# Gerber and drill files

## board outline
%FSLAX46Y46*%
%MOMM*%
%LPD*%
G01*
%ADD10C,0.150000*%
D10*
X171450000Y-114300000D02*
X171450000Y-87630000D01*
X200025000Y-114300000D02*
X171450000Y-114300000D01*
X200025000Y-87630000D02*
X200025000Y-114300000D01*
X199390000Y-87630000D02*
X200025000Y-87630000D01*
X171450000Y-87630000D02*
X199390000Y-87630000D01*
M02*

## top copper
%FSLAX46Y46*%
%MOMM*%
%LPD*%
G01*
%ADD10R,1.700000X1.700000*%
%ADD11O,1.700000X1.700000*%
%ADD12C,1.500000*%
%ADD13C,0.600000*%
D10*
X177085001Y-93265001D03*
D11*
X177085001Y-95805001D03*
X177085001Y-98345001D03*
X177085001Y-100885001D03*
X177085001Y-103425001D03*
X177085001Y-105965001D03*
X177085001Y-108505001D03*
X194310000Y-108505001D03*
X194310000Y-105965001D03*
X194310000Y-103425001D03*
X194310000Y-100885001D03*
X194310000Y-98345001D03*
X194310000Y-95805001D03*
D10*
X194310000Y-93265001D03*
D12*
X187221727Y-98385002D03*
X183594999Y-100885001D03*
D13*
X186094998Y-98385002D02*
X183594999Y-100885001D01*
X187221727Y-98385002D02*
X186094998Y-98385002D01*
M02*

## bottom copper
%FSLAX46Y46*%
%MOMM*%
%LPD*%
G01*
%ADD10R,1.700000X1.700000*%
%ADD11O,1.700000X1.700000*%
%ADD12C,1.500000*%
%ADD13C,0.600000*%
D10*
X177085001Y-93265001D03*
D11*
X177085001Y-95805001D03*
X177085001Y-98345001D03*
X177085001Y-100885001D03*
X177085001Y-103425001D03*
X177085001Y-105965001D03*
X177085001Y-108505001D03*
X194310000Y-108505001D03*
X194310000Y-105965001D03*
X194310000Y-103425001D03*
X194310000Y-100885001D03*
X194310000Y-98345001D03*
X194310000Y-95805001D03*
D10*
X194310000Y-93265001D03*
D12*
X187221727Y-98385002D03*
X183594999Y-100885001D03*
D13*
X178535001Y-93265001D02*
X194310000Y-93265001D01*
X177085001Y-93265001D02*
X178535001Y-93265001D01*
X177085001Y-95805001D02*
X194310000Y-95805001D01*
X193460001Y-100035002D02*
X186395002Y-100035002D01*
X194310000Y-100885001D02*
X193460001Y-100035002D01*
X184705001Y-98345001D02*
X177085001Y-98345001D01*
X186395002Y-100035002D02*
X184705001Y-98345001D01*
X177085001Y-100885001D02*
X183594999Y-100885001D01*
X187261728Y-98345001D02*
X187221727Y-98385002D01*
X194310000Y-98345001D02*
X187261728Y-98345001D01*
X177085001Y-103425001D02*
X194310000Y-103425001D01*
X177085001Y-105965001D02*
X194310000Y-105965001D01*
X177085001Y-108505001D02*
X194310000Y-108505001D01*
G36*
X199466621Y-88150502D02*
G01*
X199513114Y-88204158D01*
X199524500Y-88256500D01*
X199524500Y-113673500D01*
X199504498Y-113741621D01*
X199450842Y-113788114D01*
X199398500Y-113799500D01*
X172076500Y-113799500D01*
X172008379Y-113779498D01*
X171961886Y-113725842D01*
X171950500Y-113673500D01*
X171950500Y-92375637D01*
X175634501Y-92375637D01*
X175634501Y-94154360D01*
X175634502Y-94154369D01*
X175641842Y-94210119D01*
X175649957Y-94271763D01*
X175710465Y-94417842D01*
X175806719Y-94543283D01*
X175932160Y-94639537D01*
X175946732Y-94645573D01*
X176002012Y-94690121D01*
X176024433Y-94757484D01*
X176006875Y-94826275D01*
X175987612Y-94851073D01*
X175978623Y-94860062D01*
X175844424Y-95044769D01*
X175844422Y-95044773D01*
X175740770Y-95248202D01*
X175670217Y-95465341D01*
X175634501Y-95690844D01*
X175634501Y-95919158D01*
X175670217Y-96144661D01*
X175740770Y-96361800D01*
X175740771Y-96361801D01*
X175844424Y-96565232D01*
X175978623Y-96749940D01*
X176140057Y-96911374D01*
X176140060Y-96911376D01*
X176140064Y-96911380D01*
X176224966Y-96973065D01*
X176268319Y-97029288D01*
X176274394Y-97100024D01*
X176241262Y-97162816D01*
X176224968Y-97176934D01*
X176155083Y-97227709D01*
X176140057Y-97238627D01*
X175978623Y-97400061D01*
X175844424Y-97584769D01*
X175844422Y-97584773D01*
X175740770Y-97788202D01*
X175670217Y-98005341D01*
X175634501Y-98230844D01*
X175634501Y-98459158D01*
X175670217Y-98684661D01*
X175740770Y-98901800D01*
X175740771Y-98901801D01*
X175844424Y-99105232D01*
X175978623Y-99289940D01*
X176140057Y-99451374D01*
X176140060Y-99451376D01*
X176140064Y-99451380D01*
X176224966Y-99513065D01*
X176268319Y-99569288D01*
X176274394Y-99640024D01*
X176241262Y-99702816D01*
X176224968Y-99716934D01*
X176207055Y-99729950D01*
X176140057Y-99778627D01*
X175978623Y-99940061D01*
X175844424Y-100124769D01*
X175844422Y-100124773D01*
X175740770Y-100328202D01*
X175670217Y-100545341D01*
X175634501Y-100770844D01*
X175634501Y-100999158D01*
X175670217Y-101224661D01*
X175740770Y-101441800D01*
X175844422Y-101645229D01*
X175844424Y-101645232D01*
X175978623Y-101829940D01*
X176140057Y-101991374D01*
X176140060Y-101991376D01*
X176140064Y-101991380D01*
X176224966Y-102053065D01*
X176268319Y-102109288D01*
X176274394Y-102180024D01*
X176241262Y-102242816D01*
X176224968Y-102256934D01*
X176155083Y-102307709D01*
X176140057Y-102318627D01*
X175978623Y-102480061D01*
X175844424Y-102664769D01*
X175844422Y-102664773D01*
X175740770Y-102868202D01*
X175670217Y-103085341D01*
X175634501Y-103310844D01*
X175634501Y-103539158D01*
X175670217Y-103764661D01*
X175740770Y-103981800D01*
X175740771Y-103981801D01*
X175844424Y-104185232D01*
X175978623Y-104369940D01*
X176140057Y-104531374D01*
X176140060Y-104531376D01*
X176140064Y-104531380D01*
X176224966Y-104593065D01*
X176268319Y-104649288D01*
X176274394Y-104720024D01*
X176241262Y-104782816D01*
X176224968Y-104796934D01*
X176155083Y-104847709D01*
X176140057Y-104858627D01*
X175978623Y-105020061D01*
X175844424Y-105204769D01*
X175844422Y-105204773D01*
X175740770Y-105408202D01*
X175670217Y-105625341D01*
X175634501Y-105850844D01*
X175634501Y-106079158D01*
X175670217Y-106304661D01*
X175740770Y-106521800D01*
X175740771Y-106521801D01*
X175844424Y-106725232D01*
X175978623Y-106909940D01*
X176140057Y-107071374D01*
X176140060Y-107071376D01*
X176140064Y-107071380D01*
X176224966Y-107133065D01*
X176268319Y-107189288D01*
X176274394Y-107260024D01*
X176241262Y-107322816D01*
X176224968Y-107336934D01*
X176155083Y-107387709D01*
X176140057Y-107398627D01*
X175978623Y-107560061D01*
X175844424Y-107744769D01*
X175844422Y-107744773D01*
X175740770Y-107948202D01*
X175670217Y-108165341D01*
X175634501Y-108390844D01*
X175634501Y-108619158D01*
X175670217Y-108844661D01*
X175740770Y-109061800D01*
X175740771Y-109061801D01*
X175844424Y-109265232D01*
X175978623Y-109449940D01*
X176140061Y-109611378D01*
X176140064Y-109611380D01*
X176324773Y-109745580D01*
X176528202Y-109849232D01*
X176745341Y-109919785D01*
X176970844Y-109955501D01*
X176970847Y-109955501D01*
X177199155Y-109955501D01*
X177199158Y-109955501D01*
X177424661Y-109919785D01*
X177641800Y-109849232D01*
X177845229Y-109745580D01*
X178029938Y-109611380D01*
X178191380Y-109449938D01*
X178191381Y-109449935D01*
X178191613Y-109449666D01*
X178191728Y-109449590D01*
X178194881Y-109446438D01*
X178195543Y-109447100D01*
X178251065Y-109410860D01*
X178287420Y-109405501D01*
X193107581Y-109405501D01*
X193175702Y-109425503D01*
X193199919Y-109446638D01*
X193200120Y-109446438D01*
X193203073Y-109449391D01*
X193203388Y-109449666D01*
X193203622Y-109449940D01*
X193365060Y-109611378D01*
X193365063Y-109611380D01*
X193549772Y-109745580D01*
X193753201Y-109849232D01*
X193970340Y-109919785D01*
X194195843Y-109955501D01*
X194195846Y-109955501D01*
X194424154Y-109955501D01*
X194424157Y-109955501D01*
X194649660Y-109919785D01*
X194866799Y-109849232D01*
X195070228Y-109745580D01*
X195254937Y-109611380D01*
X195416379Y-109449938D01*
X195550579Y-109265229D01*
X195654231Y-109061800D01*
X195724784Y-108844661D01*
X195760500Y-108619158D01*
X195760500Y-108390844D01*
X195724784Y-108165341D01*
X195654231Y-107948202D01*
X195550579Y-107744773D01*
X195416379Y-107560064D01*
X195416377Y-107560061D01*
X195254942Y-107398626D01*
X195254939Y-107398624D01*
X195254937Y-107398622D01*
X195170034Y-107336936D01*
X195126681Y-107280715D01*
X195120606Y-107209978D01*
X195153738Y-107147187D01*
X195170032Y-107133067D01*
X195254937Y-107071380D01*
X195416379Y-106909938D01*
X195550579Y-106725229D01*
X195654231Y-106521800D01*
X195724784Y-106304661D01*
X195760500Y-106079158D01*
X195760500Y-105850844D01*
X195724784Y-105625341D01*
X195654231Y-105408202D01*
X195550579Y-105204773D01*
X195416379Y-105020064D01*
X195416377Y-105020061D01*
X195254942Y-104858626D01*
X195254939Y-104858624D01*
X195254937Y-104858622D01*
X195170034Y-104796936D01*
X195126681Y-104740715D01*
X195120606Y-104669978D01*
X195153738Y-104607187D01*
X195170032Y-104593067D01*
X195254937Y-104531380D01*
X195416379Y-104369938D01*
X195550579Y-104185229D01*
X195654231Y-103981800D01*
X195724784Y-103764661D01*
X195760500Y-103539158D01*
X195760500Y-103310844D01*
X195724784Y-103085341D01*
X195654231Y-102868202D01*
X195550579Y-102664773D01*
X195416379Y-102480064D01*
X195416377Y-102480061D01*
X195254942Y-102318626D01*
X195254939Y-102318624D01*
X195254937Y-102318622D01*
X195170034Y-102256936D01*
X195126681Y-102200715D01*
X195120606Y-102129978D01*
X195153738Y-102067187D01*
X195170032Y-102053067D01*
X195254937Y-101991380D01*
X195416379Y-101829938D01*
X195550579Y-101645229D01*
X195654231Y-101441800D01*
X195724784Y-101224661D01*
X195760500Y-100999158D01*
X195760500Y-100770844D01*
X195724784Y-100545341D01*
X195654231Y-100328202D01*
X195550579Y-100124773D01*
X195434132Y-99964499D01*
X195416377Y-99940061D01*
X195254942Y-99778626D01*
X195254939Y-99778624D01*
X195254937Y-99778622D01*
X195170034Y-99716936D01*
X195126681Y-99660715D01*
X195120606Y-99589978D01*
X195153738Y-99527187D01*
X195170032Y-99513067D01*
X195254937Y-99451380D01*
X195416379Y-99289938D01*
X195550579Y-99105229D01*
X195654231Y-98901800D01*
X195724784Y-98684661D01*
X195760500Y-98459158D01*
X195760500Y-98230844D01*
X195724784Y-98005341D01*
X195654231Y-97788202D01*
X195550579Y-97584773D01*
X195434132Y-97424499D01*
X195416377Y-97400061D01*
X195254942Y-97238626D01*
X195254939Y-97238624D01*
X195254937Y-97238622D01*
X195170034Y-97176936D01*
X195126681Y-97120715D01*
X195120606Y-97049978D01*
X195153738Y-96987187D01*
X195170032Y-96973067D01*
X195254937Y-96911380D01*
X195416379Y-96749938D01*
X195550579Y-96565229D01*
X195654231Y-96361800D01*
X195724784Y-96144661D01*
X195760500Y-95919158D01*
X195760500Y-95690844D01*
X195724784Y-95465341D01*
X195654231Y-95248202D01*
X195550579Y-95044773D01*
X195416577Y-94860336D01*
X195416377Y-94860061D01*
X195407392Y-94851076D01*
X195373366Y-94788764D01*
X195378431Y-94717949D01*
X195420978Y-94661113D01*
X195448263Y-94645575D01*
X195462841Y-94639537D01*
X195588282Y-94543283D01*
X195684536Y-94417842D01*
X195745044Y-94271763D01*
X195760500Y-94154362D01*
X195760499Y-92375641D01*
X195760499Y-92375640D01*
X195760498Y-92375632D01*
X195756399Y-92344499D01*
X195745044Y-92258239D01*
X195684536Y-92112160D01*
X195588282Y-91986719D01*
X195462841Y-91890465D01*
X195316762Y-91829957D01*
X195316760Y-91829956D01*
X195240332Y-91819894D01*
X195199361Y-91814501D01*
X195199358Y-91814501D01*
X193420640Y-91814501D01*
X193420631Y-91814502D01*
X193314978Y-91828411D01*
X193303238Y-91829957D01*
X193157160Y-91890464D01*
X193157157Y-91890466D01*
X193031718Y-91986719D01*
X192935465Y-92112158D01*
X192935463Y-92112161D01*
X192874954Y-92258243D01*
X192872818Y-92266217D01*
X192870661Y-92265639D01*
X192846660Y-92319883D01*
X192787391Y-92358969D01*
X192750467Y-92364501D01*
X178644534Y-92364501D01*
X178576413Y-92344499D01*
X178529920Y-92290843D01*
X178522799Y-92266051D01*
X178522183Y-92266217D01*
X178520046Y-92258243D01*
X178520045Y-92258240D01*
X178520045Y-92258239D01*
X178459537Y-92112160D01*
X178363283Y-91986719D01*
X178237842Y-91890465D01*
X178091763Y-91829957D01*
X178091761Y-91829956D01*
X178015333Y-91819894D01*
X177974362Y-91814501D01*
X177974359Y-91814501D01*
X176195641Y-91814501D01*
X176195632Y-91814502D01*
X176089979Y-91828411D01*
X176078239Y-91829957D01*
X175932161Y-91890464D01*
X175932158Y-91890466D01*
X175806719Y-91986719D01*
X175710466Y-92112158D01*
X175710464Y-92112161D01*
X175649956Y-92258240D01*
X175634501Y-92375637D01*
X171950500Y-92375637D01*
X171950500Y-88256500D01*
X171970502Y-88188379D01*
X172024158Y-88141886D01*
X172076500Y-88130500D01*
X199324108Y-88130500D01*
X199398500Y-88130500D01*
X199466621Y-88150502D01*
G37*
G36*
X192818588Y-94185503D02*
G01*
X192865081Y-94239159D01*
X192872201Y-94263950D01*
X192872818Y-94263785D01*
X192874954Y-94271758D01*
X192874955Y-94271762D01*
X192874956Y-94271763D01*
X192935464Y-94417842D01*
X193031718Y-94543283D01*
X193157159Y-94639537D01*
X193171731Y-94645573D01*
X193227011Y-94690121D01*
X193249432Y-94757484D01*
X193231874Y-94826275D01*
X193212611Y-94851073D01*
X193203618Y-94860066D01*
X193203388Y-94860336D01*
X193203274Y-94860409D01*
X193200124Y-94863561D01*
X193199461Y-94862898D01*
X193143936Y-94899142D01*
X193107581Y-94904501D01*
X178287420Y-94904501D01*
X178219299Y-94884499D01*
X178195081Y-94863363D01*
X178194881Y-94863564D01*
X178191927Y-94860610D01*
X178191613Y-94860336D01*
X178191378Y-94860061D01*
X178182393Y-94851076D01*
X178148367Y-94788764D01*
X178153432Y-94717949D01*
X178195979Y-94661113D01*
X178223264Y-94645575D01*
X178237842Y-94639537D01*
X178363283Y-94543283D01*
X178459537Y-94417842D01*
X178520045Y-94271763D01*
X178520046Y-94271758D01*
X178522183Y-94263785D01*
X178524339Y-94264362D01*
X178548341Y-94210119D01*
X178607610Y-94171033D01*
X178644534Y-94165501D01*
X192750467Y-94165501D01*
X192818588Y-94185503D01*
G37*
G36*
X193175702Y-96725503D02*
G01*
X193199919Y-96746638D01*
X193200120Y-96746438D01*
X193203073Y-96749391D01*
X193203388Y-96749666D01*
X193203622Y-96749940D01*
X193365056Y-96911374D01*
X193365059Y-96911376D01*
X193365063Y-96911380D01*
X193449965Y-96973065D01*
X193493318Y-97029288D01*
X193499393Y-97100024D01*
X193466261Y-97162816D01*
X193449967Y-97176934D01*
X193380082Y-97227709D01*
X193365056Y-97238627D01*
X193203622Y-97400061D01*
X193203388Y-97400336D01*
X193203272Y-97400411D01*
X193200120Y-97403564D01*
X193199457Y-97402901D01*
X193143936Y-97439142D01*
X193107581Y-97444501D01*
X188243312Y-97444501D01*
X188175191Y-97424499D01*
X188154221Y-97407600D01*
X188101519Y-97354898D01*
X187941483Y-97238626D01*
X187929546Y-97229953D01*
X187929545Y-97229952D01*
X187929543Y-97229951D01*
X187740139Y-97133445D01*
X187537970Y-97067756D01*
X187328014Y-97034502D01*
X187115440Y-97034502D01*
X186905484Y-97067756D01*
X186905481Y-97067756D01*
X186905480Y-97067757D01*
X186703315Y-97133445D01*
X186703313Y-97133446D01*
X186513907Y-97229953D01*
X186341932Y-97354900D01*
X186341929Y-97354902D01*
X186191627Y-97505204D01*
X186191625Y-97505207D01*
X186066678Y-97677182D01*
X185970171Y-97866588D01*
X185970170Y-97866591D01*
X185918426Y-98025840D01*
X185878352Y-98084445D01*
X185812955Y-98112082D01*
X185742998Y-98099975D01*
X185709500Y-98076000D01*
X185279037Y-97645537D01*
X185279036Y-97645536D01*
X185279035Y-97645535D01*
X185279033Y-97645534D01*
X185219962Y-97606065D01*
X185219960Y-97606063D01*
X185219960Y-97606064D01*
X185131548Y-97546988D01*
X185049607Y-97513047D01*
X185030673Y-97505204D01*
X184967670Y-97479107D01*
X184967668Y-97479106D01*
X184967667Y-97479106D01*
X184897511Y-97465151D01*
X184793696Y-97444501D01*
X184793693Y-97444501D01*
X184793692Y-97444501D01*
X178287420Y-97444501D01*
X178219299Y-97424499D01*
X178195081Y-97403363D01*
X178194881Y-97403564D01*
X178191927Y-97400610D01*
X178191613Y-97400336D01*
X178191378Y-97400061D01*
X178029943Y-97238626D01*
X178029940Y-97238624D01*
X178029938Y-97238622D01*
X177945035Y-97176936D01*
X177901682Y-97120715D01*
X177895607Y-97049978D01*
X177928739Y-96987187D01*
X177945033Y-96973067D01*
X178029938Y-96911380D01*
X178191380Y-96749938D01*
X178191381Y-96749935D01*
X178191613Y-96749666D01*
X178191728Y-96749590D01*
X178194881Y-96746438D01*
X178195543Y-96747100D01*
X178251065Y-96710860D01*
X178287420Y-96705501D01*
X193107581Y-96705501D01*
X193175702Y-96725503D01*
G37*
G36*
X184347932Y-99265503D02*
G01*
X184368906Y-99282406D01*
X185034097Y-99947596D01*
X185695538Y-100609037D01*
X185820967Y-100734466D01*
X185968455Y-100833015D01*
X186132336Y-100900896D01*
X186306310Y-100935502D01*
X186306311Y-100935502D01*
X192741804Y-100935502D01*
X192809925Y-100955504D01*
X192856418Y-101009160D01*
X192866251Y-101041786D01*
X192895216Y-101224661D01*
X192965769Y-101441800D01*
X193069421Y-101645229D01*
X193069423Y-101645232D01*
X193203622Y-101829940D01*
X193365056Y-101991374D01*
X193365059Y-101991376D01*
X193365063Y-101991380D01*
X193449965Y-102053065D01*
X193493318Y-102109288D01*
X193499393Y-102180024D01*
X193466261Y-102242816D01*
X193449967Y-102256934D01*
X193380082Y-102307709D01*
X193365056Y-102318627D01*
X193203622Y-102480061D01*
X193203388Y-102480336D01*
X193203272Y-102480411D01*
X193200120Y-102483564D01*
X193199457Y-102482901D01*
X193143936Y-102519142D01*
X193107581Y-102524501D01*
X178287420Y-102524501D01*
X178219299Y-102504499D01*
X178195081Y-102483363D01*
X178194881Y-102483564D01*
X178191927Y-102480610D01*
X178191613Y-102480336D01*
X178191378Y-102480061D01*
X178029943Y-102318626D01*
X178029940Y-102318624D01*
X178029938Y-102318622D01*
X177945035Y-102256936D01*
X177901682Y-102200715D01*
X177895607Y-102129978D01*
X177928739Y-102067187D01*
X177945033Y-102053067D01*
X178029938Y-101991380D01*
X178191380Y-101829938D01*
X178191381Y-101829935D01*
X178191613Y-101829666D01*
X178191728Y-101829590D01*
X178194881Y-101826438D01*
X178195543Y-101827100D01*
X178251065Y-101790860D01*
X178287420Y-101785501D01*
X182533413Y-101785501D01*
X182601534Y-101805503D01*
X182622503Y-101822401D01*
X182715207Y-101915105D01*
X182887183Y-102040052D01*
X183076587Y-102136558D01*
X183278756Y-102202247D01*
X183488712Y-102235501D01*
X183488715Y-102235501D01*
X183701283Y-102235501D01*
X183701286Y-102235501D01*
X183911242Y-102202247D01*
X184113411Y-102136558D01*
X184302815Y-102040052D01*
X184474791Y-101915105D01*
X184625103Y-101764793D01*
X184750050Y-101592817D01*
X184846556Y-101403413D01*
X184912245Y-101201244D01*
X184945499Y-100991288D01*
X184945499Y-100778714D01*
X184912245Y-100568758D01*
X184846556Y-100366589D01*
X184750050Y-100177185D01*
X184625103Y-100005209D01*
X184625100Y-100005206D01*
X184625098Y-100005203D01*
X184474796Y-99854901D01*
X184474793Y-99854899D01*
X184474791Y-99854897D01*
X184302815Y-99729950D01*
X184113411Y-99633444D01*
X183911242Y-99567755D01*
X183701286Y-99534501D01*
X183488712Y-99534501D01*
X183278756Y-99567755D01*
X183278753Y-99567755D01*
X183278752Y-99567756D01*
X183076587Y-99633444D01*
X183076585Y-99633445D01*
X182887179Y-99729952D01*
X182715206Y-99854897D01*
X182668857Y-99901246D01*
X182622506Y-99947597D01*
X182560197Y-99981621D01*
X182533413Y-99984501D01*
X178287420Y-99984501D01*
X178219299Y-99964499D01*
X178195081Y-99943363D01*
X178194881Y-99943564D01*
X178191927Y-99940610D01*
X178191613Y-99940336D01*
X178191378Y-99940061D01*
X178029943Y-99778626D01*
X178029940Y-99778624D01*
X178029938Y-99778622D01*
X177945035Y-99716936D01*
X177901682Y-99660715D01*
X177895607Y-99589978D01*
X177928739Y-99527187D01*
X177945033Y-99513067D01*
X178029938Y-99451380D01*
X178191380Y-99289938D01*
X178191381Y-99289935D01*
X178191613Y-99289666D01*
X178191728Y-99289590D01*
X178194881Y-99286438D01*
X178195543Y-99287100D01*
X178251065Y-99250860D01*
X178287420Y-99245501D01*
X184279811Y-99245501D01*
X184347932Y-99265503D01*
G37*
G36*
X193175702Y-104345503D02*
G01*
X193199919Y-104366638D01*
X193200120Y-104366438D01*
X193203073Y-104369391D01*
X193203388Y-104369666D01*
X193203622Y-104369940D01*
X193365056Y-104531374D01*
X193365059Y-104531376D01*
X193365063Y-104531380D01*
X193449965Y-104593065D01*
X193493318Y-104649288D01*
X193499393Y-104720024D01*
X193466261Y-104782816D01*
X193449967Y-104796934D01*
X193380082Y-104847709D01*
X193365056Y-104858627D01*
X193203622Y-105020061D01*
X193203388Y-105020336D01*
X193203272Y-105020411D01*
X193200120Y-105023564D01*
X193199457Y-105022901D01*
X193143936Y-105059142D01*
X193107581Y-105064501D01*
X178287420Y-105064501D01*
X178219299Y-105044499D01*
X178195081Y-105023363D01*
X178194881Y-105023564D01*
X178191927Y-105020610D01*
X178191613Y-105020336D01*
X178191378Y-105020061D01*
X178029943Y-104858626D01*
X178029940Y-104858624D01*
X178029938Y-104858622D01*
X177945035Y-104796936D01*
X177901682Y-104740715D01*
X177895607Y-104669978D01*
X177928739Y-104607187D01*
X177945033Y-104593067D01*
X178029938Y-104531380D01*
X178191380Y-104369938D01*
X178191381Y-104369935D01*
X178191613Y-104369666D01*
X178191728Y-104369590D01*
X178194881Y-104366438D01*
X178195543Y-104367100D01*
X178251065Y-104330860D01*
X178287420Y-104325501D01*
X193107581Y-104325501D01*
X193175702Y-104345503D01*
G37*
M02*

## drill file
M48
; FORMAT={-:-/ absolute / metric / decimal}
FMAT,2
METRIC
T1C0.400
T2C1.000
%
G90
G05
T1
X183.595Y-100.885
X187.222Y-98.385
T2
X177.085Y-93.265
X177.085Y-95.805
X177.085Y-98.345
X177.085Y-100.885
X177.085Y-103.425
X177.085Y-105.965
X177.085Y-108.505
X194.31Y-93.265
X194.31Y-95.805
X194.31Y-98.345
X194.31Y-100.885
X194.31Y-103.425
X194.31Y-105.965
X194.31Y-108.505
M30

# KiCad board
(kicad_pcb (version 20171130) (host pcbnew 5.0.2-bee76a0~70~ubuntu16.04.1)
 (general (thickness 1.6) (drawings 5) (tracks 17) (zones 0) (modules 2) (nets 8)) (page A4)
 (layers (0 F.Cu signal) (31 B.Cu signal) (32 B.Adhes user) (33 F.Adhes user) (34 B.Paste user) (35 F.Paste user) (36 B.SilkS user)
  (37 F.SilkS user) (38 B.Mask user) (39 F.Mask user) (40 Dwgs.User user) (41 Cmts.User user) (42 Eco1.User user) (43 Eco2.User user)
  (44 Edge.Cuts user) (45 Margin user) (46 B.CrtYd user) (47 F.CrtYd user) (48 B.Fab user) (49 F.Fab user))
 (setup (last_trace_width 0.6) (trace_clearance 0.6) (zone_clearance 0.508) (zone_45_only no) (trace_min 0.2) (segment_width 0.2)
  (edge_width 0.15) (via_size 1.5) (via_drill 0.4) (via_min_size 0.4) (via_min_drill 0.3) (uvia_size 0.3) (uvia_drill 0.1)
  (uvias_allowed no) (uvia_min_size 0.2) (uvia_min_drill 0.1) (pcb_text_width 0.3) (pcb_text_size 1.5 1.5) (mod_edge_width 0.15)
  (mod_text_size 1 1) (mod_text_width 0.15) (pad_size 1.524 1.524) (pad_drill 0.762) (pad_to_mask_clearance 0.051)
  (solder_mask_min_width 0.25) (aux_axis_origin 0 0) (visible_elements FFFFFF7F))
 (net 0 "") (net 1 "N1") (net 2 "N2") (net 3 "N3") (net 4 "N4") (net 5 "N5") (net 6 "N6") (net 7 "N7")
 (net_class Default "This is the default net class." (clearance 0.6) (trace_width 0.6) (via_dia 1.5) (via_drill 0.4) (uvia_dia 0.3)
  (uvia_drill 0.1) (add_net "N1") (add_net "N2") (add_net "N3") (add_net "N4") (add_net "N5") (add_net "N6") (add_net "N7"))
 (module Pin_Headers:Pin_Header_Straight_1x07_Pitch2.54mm (layer F.Cu) (at 177.085001 93.265001)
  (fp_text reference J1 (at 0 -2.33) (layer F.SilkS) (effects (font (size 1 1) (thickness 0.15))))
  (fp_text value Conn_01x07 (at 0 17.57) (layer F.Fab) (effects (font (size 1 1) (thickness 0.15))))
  (pad 1 thru_hole rect (at 0 0) (size 1.7 1.7) (drill 1) (layers *.Cu *.Mask) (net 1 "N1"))
  (pad 2 thru_hole oval (at 0 2.54) (size 1.7 1.7) (drill 1) (layers *.Cu *.Mask) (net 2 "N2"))
  (pad 3 thru_hole oval (at 0 5.08) (size 1.7 1.7) (drill 1) (layers *.Cu *.Mask) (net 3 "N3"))
  (pad 4 thru_hole oval (at 0 7.62) (size 1.7 1.7) (drill 1) (layers *.Cu *.Mask) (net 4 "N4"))
  (pad 5 thru_hole oval (at 0 10.16) (size 1.7 1.7) (drill 1) (layers *.Cu *.Mask) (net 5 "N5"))
  (pad 6 thru_hole oval (at 0 12.7) (size 1.7 1.7) (drill 1) (layers *.Cu *.Mask) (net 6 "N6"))
  (pad 7 thru_hole oval (at 0 15.24) (size 1.7 1.7) (drill 1) (layers *.Cu *.Mask) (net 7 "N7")))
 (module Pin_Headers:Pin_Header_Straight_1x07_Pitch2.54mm (layer F.Cu) (at 194.31 93.265001)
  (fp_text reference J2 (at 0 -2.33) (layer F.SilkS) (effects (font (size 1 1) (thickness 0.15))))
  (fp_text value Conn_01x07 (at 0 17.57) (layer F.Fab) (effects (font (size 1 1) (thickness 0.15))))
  (pad 7 thru_hole oval (at 0 15.24) (size 1.7 1.7) (drill 1) (layers *.Cu *.Mask) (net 7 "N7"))
  (pad 6 thru_hole oval (at 0 12.7) (size 1.7 1.7) (drill 1) (layers *.Cu *.Mask) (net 6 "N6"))
  (pad 5 thru_hole oval (at 0 10.16) (size 1.7 1.7) (drill 1) (layers *.Cu *.Mask) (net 5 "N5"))
  (pad 4 thru_hole oval (at 0 7.62) (size 1.7 1.7) (drill 1) (layers *.Cu *.Mask) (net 3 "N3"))
  (pad 3 thru_hole oval (at 0 5.08) (size 1.7 1.7) (drill 1) (layers *.Cu *.Mask) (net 4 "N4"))
  (pad 2 thru_hole oval (at 0 2.54) (size 1.7 1.7) (drill 1) (layers *.Cu *.Mask) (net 2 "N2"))
  (pad 1 thru_hole rect (at 0 0) (size 1.7 1.7) (drill 1) (layers *.Cu *.Mask) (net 1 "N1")))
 (gr_line (start 171.45 114.3) (end 171.45 87.63) (layer Edge.Cuts) (width 0.15))
 (gr_line (start 200.025 114.3) (end 171.45 114.3) (layer Edge.Cuts) (width 0.15))
 (gr_line (start 200.025 87.63) (end 200.025 114.3) (layer Edge.Cuts) (width 0.15))
 (gr_line (start 199.39 87.63) (end 200.025 87.63) (layer Edge.Cuts) (width 0.15))
 (gr_line (start 171.45 87.63) (end 199.39 87.63) (layer Edge.Cuts) (width 0.15))
 (segment (start 178.535001 93.265001) (end 194.31 93.265001) (width 0.6) (layer B.Cu) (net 1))
 (segment (start 177.085001 93.265001) (end 178.535001 93.265001) (width 0.6) (layer B.Cu) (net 1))
 (segment (start 177.085001 95.805001) (end 194.31 95.805001) (width 0.6) (layer B.Cu) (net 2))
 (segment (start 193.460001 100.035002) (end 186.395002 100.035002) (width 0.6) (layer B.Cu) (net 3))
 (segment (start 194.31 100.885001) (end 193.460001 100.035002) (width 0.6) (layer B.Cu) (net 3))
 (segment (start 184.705001 98.345001) (end 177.085001 98.345001) (width 0.6) (layer B.Cu) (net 3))
 (segment (start 186.395002 100.035002) (end 184.705001 98.345001) (width 0.6) (layer B.Cu) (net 3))
 (segment (start 177.085001 100.885001) (end 183.594999 100.885001) (width 0.6) (layer B.Cu) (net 4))
 (via (at 187.221727 98.385002) (size 1.5) (drill 0.4) (layers F.Cu B.Cu) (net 4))
 (segment (start 187.261728 98.345001) (end 187.221727 98.385002) (width 0.6) (layer B.Cu) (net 4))
 (segment (start 194.31 98.345001) (end 187.261728 98.345001) (width 0.6) (layer B.Cu) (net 4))
 (segment (start 186.094998 98.385002) (end 183.594999 100.885001) (width 0.6) (layer F.Cu) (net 4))
 (via (at 183.594999 100.885001) (size 1.5) (drill 0.4) (layers F.Cu B.Cu) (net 4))
 (segment (start 187.221727 98.385002) (end 186.094998 98.385002) (width 0.6) (layer F.Cu) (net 4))
 (segment (start 177.085001 103.425001) (end 194.31 103.425001) (width 0.6) (layer B.Cu) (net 5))
 (segment (start 177.085001 105.965001) (end 194.31 105.965001) (width 0.6) (layer B.Cu) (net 6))
 (segment (start 177.085001 108.505001) (end 194.31 108.505001) (width 0.6) (layer B.Cu) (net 7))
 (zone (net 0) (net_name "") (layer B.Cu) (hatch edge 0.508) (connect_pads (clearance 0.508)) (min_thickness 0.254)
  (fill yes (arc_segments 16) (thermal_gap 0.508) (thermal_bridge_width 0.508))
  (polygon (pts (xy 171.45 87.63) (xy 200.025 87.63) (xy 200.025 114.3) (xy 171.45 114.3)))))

